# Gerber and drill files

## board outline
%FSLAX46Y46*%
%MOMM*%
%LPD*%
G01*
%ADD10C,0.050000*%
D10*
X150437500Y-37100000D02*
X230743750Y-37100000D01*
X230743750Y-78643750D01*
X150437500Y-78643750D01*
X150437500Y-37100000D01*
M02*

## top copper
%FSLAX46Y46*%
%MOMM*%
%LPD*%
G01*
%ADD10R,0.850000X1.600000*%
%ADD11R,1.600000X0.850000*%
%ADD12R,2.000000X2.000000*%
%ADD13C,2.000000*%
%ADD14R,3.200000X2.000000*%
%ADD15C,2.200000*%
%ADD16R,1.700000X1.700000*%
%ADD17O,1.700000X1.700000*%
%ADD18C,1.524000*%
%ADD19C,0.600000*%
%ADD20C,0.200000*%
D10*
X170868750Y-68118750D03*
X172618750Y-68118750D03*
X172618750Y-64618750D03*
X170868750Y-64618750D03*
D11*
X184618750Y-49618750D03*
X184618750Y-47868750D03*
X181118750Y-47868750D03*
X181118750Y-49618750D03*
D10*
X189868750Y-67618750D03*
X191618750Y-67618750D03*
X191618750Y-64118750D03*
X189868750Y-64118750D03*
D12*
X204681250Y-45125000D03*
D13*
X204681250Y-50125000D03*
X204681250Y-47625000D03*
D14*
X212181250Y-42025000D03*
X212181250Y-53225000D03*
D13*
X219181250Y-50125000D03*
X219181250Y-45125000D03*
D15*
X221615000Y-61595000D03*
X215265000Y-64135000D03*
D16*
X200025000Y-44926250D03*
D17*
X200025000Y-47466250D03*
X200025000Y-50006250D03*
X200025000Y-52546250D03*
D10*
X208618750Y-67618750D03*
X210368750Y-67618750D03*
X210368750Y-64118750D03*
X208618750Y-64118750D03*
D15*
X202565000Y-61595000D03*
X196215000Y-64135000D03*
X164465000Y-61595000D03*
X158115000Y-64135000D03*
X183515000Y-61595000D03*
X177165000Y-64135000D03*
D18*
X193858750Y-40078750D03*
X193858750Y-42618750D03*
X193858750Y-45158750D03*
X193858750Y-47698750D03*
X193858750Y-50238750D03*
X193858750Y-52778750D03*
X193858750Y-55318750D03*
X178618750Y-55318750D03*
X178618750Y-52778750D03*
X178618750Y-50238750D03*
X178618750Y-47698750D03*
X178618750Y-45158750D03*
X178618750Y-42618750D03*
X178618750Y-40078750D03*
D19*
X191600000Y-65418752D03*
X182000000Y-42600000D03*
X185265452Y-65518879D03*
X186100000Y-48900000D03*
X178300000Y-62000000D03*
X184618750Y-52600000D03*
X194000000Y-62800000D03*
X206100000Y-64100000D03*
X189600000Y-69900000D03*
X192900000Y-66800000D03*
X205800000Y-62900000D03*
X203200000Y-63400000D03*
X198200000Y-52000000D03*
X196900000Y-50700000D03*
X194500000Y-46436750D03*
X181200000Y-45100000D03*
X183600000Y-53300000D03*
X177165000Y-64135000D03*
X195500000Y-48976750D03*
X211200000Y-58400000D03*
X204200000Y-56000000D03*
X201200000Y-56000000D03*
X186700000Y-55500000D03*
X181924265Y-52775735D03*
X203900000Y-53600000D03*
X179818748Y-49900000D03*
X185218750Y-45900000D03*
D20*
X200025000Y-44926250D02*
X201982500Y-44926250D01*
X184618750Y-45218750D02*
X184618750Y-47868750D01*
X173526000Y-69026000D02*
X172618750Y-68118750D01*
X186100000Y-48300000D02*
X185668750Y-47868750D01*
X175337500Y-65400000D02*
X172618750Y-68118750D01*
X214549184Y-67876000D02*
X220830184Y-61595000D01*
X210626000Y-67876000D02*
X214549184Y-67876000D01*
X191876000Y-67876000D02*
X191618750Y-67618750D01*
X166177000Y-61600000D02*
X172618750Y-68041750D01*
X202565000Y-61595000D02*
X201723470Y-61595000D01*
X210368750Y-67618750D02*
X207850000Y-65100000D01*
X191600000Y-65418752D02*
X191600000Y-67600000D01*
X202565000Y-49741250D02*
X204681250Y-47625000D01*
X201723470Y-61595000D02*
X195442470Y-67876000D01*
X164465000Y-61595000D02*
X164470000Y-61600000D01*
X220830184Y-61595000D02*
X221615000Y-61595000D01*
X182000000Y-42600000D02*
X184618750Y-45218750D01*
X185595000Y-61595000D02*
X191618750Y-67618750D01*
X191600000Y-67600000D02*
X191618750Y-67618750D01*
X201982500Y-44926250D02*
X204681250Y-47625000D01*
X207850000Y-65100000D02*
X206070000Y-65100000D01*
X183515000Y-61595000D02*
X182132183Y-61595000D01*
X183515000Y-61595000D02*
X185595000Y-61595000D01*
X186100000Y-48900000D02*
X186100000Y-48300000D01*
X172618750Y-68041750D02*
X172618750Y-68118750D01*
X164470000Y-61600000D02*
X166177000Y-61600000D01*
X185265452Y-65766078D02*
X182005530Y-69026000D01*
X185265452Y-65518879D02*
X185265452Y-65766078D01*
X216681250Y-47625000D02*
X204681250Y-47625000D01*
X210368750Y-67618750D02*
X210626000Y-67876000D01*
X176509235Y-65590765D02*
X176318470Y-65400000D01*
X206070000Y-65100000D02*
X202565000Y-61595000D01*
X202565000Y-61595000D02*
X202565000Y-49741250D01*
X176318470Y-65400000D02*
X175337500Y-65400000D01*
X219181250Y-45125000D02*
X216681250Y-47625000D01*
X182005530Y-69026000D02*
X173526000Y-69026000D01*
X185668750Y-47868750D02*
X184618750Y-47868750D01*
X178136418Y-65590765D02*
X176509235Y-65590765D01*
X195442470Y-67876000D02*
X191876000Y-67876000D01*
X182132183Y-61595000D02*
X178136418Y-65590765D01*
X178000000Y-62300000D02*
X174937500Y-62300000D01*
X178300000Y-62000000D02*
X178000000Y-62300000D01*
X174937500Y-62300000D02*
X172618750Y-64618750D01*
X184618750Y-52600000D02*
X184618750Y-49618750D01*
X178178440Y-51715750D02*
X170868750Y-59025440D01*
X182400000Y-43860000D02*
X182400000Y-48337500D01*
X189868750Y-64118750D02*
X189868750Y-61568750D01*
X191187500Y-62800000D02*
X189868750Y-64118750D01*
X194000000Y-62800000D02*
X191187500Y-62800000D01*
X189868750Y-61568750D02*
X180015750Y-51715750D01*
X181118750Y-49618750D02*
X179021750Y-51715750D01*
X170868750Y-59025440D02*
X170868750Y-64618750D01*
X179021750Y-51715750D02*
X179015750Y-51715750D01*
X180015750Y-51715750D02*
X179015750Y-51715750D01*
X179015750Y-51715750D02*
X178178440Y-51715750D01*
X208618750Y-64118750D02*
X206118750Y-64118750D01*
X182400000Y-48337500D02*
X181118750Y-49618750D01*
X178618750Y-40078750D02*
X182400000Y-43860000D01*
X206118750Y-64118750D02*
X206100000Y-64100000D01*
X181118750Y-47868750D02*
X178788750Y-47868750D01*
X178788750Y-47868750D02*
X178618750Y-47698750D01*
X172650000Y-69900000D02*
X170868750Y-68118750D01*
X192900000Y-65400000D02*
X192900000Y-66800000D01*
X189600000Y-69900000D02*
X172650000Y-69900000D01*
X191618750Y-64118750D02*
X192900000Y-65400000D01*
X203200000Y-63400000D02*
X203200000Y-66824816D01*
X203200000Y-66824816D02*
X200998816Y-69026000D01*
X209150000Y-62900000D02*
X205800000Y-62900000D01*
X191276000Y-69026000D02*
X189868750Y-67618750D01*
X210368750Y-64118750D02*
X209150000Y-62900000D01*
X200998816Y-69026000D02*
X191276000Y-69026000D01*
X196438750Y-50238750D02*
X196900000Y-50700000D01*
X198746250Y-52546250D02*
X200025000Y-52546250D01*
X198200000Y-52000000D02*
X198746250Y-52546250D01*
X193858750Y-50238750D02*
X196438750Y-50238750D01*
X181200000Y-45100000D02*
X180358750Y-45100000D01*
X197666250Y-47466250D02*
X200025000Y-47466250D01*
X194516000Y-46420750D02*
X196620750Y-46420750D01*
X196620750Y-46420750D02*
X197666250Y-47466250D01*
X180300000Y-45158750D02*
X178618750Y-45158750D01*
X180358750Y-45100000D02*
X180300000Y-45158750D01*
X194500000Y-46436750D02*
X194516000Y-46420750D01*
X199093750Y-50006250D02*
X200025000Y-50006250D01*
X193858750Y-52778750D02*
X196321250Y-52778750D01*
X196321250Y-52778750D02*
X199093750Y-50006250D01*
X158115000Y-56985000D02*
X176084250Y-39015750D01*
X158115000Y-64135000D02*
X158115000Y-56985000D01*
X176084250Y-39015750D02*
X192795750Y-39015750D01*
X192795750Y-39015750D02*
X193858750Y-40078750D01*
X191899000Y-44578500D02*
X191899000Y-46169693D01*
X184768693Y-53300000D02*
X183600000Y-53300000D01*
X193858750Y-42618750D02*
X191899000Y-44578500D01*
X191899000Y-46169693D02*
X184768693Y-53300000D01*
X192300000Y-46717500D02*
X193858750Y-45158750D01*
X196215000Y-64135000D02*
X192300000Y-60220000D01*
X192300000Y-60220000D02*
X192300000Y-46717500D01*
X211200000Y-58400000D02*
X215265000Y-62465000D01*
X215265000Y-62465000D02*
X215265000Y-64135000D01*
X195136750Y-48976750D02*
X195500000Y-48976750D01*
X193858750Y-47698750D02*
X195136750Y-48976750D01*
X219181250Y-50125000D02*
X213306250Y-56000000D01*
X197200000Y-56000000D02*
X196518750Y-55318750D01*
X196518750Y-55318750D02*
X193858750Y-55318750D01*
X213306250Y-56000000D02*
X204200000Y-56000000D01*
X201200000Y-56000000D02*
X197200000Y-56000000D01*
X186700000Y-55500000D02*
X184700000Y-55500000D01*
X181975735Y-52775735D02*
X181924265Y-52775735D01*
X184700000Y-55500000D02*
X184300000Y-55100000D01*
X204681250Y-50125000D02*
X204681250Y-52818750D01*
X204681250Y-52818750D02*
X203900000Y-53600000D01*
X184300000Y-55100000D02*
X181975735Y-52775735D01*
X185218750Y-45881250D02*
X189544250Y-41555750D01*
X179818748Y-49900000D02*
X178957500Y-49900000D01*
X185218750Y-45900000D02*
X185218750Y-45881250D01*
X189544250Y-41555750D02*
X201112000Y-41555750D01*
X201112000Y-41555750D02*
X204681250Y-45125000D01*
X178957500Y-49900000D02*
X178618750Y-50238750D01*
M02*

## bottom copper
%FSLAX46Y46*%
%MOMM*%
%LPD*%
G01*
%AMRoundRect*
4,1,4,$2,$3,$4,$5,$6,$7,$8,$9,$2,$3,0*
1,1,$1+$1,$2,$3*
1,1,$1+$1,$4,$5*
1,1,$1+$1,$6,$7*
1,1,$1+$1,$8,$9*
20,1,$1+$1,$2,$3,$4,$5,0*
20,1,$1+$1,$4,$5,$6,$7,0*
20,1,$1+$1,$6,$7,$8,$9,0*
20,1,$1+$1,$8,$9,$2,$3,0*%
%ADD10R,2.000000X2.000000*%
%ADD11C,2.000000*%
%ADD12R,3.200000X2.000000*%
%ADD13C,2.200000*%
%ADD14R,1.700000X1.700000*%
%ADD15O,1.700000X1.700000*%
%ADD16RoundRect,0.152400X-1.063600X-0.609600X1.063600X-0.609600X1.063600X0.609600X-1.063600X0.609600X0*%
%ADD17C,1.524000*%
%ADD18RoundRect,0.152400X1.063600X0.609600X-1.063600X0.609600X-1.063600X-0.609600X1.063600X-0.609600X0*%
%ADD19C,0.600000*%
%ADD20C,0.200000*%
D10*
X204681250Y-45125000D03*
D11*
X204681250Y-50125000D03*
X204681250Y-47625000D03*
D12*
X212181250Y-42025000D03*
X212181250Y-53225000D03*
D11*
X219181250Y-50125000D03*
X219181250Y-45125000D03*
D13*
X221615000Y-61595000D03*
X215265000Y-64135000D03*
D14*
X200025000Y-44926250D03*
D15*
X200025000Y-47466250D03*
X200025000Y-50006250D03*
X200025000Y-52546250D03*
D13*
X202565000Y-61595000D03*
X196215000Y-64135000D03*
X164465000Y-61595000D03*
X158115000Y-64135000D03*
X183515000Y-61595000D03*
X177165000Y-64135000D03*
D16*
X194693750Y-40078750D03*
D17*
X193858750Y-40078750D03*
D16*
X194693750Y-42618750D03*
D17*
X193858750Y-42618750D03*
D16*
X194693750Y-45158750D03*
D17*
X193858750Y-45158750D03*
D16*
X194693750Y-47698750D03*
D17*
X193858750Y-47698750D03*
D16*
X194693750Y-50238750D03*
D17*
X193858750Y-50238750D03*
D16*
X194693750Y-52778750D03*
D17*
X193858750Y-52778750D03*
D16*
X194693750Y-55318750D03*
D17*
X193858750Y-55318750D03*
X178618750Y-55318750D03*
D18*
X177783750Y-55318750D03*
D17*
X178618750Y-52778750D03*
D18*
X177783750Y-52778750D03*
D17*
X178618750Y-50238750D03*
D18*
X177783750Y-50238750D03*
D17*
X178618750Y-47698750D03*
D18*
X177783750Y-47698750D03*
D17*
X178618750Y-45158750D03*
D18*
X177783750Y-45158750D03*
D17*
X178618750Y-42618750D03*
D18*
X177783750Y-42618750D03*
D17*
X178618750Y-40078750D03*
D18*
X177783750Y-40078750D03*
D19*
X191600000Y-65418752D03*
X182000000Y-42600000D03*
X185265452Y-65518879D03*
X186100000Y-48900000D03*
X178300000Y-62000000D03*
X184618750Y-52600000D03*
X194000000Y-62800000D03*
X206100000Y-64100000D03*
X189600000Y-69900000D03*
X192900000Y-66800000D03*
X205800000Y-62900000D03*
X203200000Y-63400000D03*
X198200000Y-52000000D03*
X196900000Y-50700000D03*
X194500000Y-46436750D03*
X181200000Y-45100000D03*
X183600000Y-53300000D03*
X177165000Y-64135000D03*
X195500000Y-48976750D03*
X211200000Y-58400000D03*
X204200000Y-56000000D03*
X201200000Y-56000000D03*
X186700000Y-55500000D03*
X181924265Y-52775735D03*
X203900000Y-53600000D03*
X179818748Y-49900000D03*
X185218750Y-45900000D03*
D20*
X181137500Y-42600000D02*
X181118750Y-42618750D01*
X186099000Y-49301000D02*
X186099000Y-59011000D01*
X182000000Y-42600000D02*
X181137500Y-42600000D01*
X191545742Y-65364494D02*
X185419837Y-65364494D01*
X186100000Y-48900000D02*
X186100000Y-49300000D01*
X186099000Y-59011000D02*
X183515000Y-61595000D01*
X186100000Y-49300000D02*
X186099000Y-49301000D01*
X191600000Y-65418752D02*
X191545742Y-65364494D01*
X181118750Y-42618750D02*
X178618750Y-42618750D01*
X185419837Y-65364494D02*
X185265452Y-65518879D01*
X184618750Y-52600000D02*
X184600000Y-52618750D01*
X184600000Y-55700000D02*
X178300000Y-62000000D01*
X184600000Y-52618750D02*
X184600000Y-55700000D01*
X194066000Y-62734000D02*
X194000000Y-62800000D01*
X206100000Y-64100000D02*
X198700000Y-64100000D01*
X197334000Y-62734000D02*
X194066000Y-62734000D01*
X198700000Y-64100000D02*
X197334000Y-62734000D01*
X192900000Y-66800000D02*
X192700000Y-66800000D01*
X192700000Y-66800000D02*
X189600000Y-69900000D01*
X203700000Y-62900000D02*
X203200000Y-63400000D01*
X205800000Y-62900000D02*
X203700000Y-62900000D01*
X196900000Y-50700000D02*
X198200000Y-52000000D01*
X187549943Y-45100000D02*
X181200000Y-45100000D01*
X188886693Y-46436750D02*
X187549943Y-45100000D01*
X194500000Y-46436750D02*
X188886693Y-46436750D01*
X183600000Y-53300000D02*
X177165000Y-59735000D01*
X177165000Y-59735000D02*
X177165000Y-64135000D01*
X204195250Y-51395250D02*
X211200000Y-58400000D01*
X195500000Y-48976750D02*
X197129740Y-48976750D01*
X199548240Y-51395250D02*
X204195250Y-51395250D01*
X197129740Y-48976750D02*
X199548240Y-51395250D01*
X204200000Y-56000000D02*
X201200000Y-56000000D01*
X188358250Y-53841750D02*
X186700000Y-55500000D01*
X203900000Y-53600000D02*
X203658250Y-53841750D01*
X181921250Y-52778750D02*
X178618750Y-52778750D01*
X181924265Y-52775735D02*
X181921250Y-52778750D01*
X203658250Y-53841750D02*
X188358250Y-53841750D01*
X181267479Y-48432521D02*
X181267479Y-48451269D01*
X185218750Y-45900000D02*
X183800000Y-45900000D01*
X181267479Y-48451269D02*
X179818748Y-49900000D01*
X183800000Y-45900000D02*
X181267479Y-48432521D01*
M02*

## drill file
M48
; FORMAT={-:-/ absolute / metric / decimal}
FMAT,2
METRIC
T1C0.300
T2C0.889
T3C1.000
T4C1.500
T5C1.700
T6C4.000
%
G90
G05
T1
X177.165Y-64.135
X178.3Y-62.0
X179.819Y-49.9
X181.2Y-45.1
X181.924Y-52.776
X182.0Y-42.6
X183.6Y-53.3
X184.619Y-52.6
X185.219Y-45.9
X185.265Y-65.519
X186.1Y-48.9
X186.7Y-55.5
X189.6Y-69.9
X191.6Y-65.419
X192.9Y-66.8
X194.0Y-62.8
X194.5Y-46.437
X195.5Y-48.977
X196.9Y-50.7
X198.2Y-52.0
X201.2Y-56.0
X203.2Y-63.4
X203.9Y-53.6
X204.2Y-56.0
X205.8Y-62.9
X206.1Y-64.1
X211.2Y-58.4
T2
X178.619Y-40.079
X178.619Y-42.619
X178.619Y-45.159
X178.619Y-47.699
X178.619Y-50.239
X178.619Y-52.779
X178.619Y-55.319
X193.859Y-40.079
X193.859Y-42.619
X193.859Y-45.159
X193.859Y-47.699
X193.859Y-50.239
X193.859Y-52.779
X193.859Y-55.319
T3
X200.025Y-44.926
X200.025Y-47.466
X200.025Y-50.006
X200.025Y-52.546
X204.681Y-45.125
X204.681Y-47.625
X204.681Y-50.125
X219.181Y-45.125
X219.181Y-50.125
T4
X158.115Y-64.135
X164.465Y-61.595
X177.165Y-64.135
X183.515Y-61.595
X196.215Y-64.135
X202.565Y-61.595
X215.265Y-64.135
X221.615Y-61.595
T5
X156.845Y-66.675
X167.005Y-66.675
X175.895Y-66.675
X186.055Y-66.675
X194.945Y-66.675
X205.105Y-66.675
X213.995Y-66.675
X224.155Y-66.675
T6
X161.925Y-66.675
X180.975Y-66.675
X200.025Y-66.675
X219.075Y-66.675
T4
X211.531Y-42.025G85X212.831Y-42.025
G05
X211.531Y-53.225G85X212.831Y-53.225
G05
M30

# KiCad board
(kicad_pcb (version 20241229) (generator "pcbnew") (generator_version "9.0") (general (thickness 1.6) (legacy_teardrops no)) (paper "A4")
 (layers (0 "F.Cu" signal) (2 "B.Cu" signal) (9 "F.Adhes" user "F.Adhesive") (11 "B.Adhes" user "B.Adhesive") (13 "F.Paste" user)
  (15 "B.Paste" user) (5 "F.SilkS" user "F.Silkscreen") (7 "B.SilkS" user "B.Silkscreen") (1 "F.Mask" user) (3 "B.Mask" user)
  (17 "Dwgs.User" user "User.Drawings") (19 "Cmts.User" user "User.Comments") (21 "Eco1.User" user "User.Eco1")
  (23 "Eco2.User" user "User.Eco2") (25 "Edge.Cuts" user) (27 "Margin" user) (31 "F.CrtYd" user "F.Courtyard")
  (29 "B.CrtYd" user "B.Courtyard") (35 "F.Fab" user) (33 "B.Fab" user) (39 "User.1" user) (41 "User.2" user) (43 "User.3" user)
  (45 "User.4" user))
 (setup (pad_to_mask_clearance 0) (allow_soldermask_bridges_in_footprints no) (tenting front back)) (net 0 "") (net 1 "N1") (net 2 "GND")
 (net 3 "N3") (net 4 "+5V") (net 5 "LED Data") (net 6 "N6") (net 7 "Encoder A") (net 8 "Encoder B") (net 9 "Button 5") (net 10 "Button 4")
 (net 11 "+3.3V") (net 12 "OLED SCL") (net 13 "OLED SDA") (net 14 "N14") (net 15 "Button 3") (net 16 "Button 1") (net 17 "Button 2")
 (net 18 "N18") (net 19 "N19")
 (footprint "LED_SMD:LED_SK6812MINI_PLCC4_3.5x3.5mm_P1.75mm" (layer "F.Cu") (at 171.74375 66.36875 90)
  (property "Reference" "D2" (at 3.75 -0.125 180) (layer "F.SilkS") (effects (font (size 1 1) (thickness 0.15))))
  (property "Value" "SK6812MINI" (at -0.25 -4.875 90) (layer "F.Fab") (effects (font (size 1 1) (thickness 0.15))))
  (pad "1" smd rect (at -1.75 -0.875 90) (size 1.6 0.85) (layers "F.Cu" "F.Mask" "F.Paste") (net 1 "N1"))
  (pad "2" smd rect (at -1.75 0.875 90) (size 1.6 0.85) (layers "F.Cu" "F.Mask" "F.Paste") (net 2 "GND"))
  (pad "3" smd rect (at 1.75 0.875 90) (size 1.6 0.85) (layers "F.Cu" "F.Mask" "F.Paste") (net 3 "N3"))
  (pad "4" smd rect (at 1.75 -0.875 90) (size 1.6 0.85) (layers "F.Cu" "F.Mask" "F.Paste") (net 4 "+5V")))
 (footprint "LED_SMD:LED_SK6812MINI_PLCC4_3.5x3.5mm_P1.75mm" (layer "F.Cu") (at 182.86875 48.74375 180)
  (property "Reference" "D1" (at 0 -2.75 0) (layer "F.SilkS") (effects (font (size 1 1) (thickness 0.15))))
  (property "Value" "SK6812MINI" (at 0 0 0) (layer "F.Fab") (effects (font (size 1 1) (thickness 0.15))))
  (pad "1" smd rect (at -1.75 -0.875 180) (size 1.6 0.85) (layers "F.Cu" "F.Mask" "F.Paste") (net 3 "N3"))
  (pad "2" smd rect (at -1.75 0.875 180) (size 1.6 0.85) (layers "F.Cu" "F.Mask" "F.Paste") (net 2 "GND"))
  (pad "3" smd rect (at 1.75 0.875 180) (size 1.6 0.85) (layers "F.Cu" "F.Mask" "F.Paste") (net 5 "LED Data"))
  (pad "4" smd rect (at 1.75 -0.875 180) (size 1.6 0.85) (layers "F.Cu" "F.Mask" "F.Paste") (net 4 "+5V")))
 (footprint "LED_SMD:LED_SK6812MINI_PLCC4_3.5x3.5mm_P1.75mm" (layer "F.Cu") (at 190.74375 65.86875 90)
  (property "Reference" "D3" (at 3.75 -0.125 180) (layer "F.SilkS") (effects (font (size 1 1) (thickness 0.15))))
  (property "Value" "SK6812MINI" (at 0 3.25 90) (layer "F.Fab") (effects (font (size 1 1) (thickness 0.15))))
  (pad "1" smd rect (at -1.75 -0.875 90) (size 1.6 0.85) (layers "F.Cu" "F.Mask" "F.Paste") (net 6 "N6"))
  (pad "2" smd rect (at -1.75 0.875 90) (size 1.6 0.85) (layers "F.Cu" "F.Mask" "F.Paste") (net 2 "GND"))
  (pad "3" smd rect (at 1.75 0.875 90) (size 1.6 0.85) (layers "F.Cu" "F.Mask" "F.Paste") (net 1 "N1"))
  (pad "4" smd rect (at 1.75 -0.875 90) (size 1.6 0.85) (layers "F.Cu" "F.Mask" "F.Paste") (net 4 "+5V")))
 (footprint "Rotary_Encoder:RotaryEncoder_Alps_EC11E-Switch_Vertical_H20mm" (layer "F.Cu") (at 204.68125 45.125)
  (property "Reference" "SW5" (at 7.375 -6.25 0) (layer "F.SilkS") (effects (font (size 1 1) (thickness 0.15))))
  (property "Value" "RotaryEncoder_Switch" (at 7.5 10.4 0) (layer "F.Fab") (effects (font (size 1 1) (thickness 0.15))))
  (pad "A" thru_hole rect (at 0 0) (size 2 2) (drill 1) (layers "*.Cu" "*.Mask") (remove_unused_layers no) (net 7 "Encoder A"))
  (pad "B" thru_hole circle (at 0 5) (size 2 2) (drill 1) (layers "*.Cu" "*.Mask") (remove_unused_layers no) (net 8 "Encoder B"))
  (pad "C" thru_hole circle (at 0 2.5) (size 2 2) (drill 1) (layers "*.Cu" "*.Mask") (remove_unused_layers no) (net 2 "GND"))
  (pad "MP" thru_hole rect (at 7.5 -3.1) (size 3.2 2) (drill oval 2.8 1.5) (layers "*.Cu" "*.Mask") (remove_unused_layers no))
  (pad "MP" thru_hole rect (at 7.5 8.1) (size 3.2 2) (drill oval 2.8 1.5) (layers "*.Cu" "*.Mask") (remove_unused_layers no))
  (pad "S1" thru_hole circle (at 14.5 5) (size 2 2) (drill 1) (layers "*.Cu" "*.Mask") (remove_unused_layers no) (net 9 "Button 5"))
  (pad "S2" thru_hole circle (at 14.5 0) (size 2 2) (drill 1) (layers "*.Cu" "*.Mask") (remove_unused_layers no) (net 2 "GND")))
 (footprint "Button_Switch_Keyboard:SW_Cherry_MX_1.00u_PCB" (layer "F.Cu") (at 221.615 61.595)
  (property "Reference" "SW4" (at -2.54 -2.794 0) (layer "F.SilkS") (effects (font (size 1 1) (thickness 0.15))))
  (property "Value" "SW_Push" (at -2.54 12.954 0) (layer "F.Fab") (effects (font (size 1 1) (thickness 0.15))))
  (pad "" np_thru_hole circle (at -7.62 5.08) (size 1.7 1.7) (drill 1.7) (layers "*.Cu" "*.Mask"))
  (pad "" np_thru_hole circle (at -2.54 5.08) (size 4 4) (drill 4) (layers "*.Cu" "*.Mask"))
  (pad "" np_thru_hole circle (at 2.54 5.08) (size 1.7 1.7) (drill 1.7) (layers "*.Cu" "*.Mask"))
  (pad "1" thru_hole circle (at 0 0) (size 2.2 2.2) (drill 1.5) (layers "*.Cu" "*.Mask") (remove_unused_layers no) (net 2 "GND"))
  (pad "2" thru_hole circle (at -6.35 2.54) (size 2.2 2.2) (drill 1.5) (layers "*.Cu" "*.Mask") (remove_unused_layers no)
   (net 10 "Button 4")))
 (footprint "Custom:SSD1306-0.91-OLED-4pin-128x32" (layer "F.Cu") (at 163.525 42.73625)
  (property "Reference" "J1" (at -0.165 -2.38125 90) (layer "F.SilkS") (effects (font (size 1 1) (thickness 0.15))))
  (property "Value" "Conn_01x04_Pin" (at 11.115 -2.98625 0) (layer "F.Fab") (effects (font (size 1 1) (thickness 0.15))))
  (pad "1" thru_hole rect (at 36.5 2.19) (size 1.7 1.7) (drill 1) (layers "*.Cu" "*.Mask") (remove_unused_layers no) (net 2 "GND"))
  (pad "2" thru_hole oval (at 36.5 4.73) (size 1.7 1.7) (drill 1) (layers "*.Cu" "*.Mask") (remove_unused_layers no) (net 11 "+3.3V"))
  (pad "3" thru_hole oval (at 36.5 7.27) (size 1.7 1.7) (drill 1) (layers "*.Cu" "*.Mask") (remove_unused_layers no) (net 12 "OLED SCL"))
  (pad "4" thru_hole oval (at 36.5 9.81) (size 1.7 1.7) (drill 1) (layers "*.Cu" "*.Mask") (remove_unused_layers no) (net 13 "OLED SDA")))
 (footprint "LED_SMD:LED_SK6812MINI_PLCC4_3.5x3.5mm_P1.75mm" (layer "F.Cu") (at 209.49375 65.86875 90)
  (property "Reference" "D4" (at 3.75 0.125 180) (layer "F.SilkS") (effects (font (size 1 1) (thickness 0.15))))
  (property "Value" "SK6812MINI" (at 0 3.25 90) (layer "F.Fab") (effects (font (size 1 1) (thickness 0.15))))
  (pad "1" smd rect (at -1.75 -0.875 90) (size 1.6 0.85) (layers "F.Cu" "F.Mask" "F.Paste") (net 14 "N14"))
  (pad "2" smd rect (at -1.75 0.875 90) (size 1.6 0.85) (layers "F.Cu" "F.Mask" "F.Paste") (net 2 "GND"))
  (pad "3" smd rect (at 1.75 0.875 90) (size 1.6 0.85) (layers "F.Cu" "F.Mask" "F.Paste") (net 6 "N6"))
  (pad "4" smd rect (at 1.75 -0.875 90) (size 1.6 0.85) (layers "F.Cu" "F.Mask" "F.Paste") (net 4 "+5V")))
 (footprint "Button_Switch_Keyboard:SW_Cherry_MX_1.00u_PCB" (layer "F.Cu") (at 202.565 61.595)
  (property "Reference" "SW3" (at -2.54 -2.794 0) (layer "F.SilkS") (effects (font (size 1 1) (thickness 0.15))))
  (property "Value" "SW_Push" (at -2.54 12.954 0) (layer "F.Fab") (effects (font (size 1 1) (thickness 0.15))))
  (pad "" np_thru_hole circle (at -7.62 5.08) (size 1.7 1.7) (drill 1.7) (layers "*.Cu" "*.Mask"))
  (pad "" np_thru_hole circle (at -2.54 5.08) (size 4 4) (drill 4) (layers "*.Cu" "*.Mask"))
  (pad "" np_thru_hole circle (at 2.54 5.08) (size 1.7 1.7) (drill 1.7) (layers "*.Cu" "*.Mask"))
  (pad "1" thru_hole circle (at 0 0) (size 2.2 2.2) (drill 1.5) (layers "*.Cu" "*.Mask") (remove_unused_layers no) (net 2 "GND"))
  (pad "2" thru_hole circle (at -6.35 2.54) (size 2.2 2.2) (drill 1.5) (layers "*.Cu" "*.Mask") (remove_unused_layers no)
   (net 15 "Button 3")))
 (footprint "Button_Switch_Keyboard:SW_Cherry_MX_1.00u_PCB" (layer "F.Cu") (at 164.465 61.595)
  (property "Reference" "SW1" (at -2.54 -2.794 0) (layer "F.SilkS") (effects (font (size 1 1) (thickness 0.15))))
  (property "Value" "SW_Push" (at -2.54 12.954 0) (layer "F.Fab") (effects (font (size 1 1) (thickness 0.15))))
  (pad "" np_thru_hole circle (at -7.62 5.08) (size 1.7 1.7) (drill 1.7) (layers "*.Cu" "*.Mask"))
  (pad "" np_thru_hole circle (at -2.54 5.08) (size 4 4) (drill 4) (layers "*.Cu" "*.Mask"))
  (pad "" np_thru_hole circle (at 2.54 5.08) (size 1.7 1.7) (drill 1.7) (layers "*.Cu" "*.Mask"))
  (pad "1" thru_hole circle (at 0 0) (size 2.2 2.2) (drill 1.5) (layers "*.Cu" "*.Mask") (remove_unused_layers no) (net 2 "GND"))
  (pad "2" thru_hole circle (at -6.35 2.54) (size 2.2 2.2) (drill 1.5) (layers "*.Cu" "*.Mask") (remove_unused_layers no)
   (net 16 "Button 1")))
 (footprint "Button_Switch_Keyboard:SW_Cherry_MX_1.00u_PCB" (layer "F.Cu") (at 183.515 61.595)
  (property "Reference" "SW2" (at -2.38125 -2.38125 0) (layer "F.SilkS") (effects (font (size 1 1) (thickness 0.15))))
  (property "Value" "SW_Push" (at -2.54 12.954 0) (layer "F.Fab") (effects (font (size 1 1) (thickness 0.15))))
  (pad "" np_thru_hole circle (at -7.62 5.08) (size 1.7 1.7) (drill 1.7) (layers "*.Cu" "*.Mask"))
  (pad "" np_thru_hole circle (at -2.54 5.08) (size 4 4) (drill 4) (layers "*.Cu" "*.Mask"))
  (pad "" np_thru_hole circle (at 2.54 5.08) (size 1.7 1.7) (drill 1.7) (layers "*.Cu" "*.Mask"))
  (pad "1" thru_hole circle (at 0 0) (size 2.2 2.2) (drill 1.5) (layers "*.Cu" "*.Mask") (remove_unused_layers no) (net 2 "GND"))
  (pad "2" thru_hole circle (at -6.35 2.54) (size 2.2 2.2) (drill 1.5) (layers "*.Cu" "*.Mask") (remove_unused_layers no)
   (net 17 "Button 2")))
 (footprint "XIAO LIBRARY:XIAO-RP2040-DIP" (layer "B.Cu") (at 186.23875 47.69875 180)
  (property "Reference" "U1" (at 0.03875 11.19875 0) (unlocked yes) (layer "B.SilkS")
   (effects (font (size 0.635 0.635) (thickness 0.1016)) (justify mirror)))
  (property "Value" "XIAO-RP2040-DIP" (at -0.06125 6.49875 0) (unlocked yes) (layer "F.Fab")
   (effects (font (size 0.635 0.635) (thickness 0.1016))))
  (pad "1" smd roundrect (at -8.455 7.62) (size 2.432 1.524) (layers "B.Cu" "B.Mask") (roundrect_rratio 0.1) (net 16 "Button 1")
   (thermal_bridge_angle 45))
  (pad "1" thru_hole circle (at -7.62 7.62) (size 1.524 1.524) (drill 0.889) (layers "*.Cu" "*.Mask") (remove_unused_layers no)
   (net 16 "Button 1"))
  (pad "2" smd roundrect (at -8.455 5.08) (size 2.432 1.524) (layers "B.Cu" "B.Mask") (roundrect_rratio 0.1) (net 17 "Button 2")
   (thermal_bridge_angle 45))
  (pad "2" thru_hole circle (at -7.62 5.08) (size 1.524 1.524) (drill 0.889) (layers "*.Cu" "*.Mask") (remove_unused_layers no)
   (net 17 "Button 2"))
  (pad "3" smd roundrect (at -8.455 2.54) (size 2.432 1.524) (layers "B.Cu" "B.Mask") (roundrect_rratio 0.1) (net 15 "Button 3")
   (thermal_bridge_angle 45))
  (pad "3" thru_hole circle (at -7.62 2.54) (size 1.524 1.524) (drill 0.889) (layers "*.Cu" "*.Mask") (remove_unused_layers no)
   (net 15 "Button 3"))
  (pad "4" smd roundrect (at -8.455 0) (size 2.432 1.524) (layers "B.Cu" "B.Mask") (roundrect_rratio 0.1) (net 10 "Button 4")
   (thermal_bridge_angle 45))
  (pad "4" thru_hole circle (at -7.62 0) (size 1.524 1.524) (drill 0.889) (layers "*.Cu" "*.Mask") (remove_unused_layers no)
   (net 10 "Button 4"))
  (pad "5" smd roundrect (at -8.455 -2.54) (size 2.432 1.524) (layers "B.Cu" "B.Mask") (roundrect_rratio 0.1) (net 13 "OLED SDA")
   (thermal_bridge_angle 45))
  (pad "5" thru_hole circle (at -7.62 -2.54) (size 1.524 1.524) (drill 0.889) (layers "*.Cu" "*.Mask") (remove_unused_layers no)
   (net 13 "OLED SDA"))
  (pad "6" smd roundrect (at -8.455 -5.08) (size 2.432 1.524) (layers "B.Cu" "B.Mask") (roundrect_rratio 0.1) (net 12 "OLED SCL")
   (thermal_bridge_angle 45))
  (pad "6" thru_hole circle (at -7.62 -5.08) (size 1.524 1.524) (drill 0.889) (layers "*.Cu" "*.Mask") (remove_unused_layers no)
   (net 12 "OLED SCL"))
  (pad "7" smd roundrect (at -8.455 -7.62) (size 2.432 1.524) (layers "B.Cu" "B.Mask") (roundrect_rratio 0.1) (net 9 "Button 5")
   (thermal_bridge_angle 45))
  (pad "7" thru_hole circle (at -7.62 -7.62) (size 1.524 1.524) (drill 0.889) (layers "*.Cu" "*.Mask") (remove_unused_layers no)
   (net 9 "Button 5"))
  (pad "8" thru_hole circle (at 7.62 -7.62 180) (size 1.524 1.524) (drill 0.889) (layers "*.Cu" "*.Mask") (remove_unused_layers no)
   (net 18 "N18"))
  (pad "8" smd roundrect (at 8.455 -7.62 180) (size 2.432 1.524) (layers "B.Cu" "B.Mask") (roundrect_rratio 0.1) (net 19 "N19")
   (thermal_bridge_angle 45))
  (pad "9" thru_hole circle (at 7.62 -5.08 180) (size 1.524 1.524) (drill 0.889) (layers "*.Cu" "*.Mask") (remove_unused_layers no)
   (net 8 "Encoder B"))
  (pad "9" smd roundrect (at 8.455 -5.08 180) (size 2.432 1.524) (layers "B.Cu" "B.Mask") (roundrect_rratio 0.1) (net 8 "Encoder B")
   (thermal_bridge_angle 45))
  (pad "10" thru_hole circle (at 7.62 -2.54 180) (size 1.524 1.524) (drill 0.889) (layers "*.Cu" "*.Mask") (remove_unused_layers no)
   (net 7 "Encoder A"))
  (pad "10" smd roundrect (at 8.455 -2.54 180) (size 2.432 1.524) (layers "B.Cu" "B.Mask") (roundrect_rratio 0.1) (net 7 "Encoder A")
   (thermal_bridge_angle 45))
  (pad "11" thru_hole circle (at 7.62 0 180) (size 1.524 1.524) (drill 0.889) (layers "*.Cu" "*.Mask") (remove_unused_layers no)
   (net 5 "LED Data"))
  (pad "11" smd roundrect (at 8.455 0 180) (size 2.432 1.524) (layers "B.Cu" "B.Mask") (roundrect_rratio 0.1) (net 5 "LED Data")
   (thermal_bridge_angle 45))
  (pad "12" thru_hole circle (at 7.62 2.54 180) (size 1.524 1.524) (drill 0.889) (layers "*.Cu" "*.Mask") (remove_unused_layers no)
   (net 11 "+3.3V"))
  (pad "12" smd roundrect (at 8.455 2.54 180) (size 2.432 1.524) (layers "B.Cu" "B.Mask") (roundrect_rratio 0.1) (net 11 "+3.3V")
   (thermal_bridge_angle 45))
  (pad "13" thru_hole circle (at 7.62 5.08 180) (size 1.524 1.524) (drill 0.889) (layers "*.Cu" "*.Mask") (remove_unused_layers no)
   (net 2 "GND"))
  (pad "13" smd roundrect (at 8.455 5.08 180) (size 2.432 1.524) (layers "B.Cu" "B.Mask") (roundrect_rratio 0.1) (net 2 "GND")
   (thermal_bridge_angle 45))
  (pad "14" thru_hole circle (at 7.62 7.62 180) (size 1.524 1.524) (drill 0.889) (layers "*.Cu" "*.Mask") (remove_unused_layers no)
   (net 4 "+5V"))
  (pad "14" smd roundrect (at 8.455 7.62 180) (size 2.432 1.524) (layers "B.Cu" "B.Mask") (roundrect_rratio 0.1) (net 4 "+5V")
   (thermal_bridge_angle 45)))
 (gr_rect (start 150.4375 37.1) (end 230.74375 78.64375) (stroke (width 0.05) (type default)) (fill no) (layer "Edge.Cuts"))
 (segment (start 200.025 44.92625) (end 201.9825 44.92625) (width 0.2) (layer "F.Cu") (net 2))
 (segment (start 184.61875 45.21875) (end 184.61875 47.86875) (width 0.2) (layer "F.Cu") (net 2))
 (segment (start 173.526 69.026) (end 172.61875 68.11875) (width 0.2) (layer "F.Cu") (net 2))
 (segment (start 186.1 48.3) (end 185.66875 47.86875) (width 0.2) (layer "F.Cu") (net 2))
 (segment (start 175.3375 65.4) (end 172.61875 68.11875) (width 0.2) (layer "F.Cu") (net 2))
 (segment (start 214.549184 67.876) (end 220.830184 61.595) (width 0.2) (layer "F.Cu") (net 2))
 (segment (start 210.626 67.876) (end 214.549184 67.876) (width 0.2) (layer "F.Cu") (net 2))
 (segment (start 191.876 67.876) (end 191.61875 67.61875) (width 0.2) (layer "F.Cu") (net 2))
 (segment (start 166.177 61.6) (end 172.61875 68.04175) (width 0.2) (layer "F.Cu") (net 2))
 (segment (start 202.565 61.595) (end 201.72347 61.595) (width 0.2) (layer "F.Cu") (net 2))
 (segment (start 210.36875 67.61875) (end 207.85 65.1) (width 0.2) (layer "F.Cu") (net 2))
 (segment (start 191.6 65.418752) (end 191.6 67.6) (width 0.2) (layer "F.Cu") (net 2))
 (segment (start 202.565 49.74125) (end 204.68125 47.625) (width 0.2) (layer "F.Cu") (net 2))
 (segment (start 201.72347 61.595) (end 195.44247 67.876) (width 0.2) (layer "F.Cu") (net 2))
 (segment (start 164.465 61.595) (end 164.47 61.6) (width 0.2) (layer "F.Cu") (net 2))
 (segment (start 220.830184 61.595) (end 221.615 61.595) (width 0.2) (layer "F.Cu") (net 2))
 (segment (start 182 42.6) (end 184.61875 45.21875) (width 0.2) (layer "F.Cu") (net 2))
 (segment (start 185.595 61.595) (end 191.61875 67.61875) (width 0.2) (layer "F.Cu") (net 2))
 (segment (start 191.6 67.6) (end 191.61875 67.61875) (width 0.2) (layer "F.Cu") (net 2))
 (segment (start 201.9825 44.92625) (end 204.68125 47.625) (width 0.2) (layer "F.Cu") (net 2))
 (segment (start 207.85 65.1) (end 206.07 65.1) (width 0.2) (layer "F.Cu") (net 2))
 (segment (start 183.515 61.595) (end 182.132183 61.595) (width 0.2) (layer "F.Cu") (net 2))
 (segment (start 183.515 61.595) (end 185.595 61.595) (width 0.2) (layer "F.Cu") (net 2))
 (segment (start 186.1 48.9) (end 186.1 48.3) (width 0.2) (layer "F.Cu") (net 2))
 (segment (start 172.61875 68.04175) (end 172.61875 68.11875) (width 0.2) (layer "F.Cu") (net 2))
 (segment (start 164.47 61.6) (end 166.177 61.6) (width 0.2) (layer "F.Cu") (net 2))
 (segment (start 185.265452 65.766078) (end 182.00553 69.026) (width 0.2) (layer "F.Cu") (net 2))
 (segment (start 185.265452 65.518879) (end 185.265452 65.766078) (width 0.2) (layer "F.Cu") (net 2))
 (segment (start 216.68125 47.625) (end 204.68125 47.625) (width 0.2) (layer "F.Cu") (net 2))
 (segment (start 210.36875 67.61875) (end 210.626 67.876) (width 0.2) (layer "F.Cu") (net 2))
 (segment (start 176.509235 65.590765) (end 176.31847 65.4) (width 0.2) (layer "F.Cu") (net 2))
 (segment (start 206.07 65.1) (end 202.565 61.595) (width 0.2) (layer "F.Cu") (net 2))
 (segment (start 202.565 61.595) (end 202.565 49.74125) (width 0.2) (layer "F.Cu") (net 2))
 (segment (start 176.31847 65.4) (end 175.3375 65.4) (width 0.2) (layer "F.Cu") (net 2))
 (segment (start 219.18125 45.125) (end 216.68125 47.625) (width 0.2) (layer "F.Cu") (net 2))
 (segment (start 182.00553 69.026) (end 173.526 69.026) (width 0.2) (layer "F.Cu") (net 2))
 (segment (start 185.66875 47.86875) (end 184.61875 47.86875) (width 0.2) (layer "F.Cu") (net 2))
 (segment (start 178.136418 65.590765) (end 176.509235 65.590765) (width 0.2) (layer "F.Cu") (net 2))
 (segment (start 195.44247 67.876) (end 191.876 67.876) (width 0.2) (layer "F.Cu") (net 2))
 (segment (start 182.132183 61.595) (end 178.136418 65.590765) (width 0.2) (layer "F.Cu") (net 2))
 (via (at 191.6 65.418752) (size 0.6) (drill 0.3) (layers "F.Cu" "B.Cu") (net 2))
 (via (at 182 42.6) (size 0.6) (drill 0.3) (layers "F.Cu" "B.Cu") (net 2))
 (via (at 185.265452 65.518879) (size 0.6) (drill 0.3) (layers "F.Cu" "B.Cu") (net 2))
 (via (at 186.1 48.9) (size 0.6) (drill 0.3) (layers "F.Cu" "B.Cu") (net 2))
 (segment (start 181.1375 42.6) (end 181.11875 42.61875) (width 0.2) (layer "B.Cu") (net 2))
 (segment (start 186.099 49.301) (end 186.099 59.011) (width 0.2) (layer "B.Cu") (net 2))
 (segment (start 182 42.6) (end 181.1375 42.6) (width 0.2) (layer "B.Cu") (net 2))
 (segment (start 191.545742 65.364494) (end 185.419837 65.364494) (width 0.2) (layer "B.Cu") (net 2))
 (segment (start 186.1 48.9) (end 186.1 49.3) (width 0.2) (layer "B.Cu") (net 2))
 (segment (start 186.099 59.011) (end 183.515 61.595) (width 0.2) (layer "B.Cu") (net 2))
 (segment (start 186.1 49.3) (end 186.099 49.301) (width 0.2) (layer "B.Cu") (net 2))
 (segment (start 191.6 65.418752) (end 191.545742 65.364494) (width 0.2) (layer "B.Cu") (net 2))
 (segment (start 181.11875 42.61875) (end 178.61875 42.61875) (width 0.2) (layer "B.Cu") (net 2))
 (segment (start 185.419837 65.364494) (end 185.265452 65.518879) (width 0.2) (layer "B.Cu") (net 2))
 (segment (start 178 62.3) (end 174.9375 62.3) (width 0.2) (layer "F.Cu") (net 3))
 (segment (start 178.3 62) (end 178 62.3) (width 0.2) (layer "F.Cu") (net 3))
 (segment (start 174.9375 62.3) (end 172.61875 64.61875) (width 0.2) (layer "F.Cu") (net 3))
 (segment (start 184.61875 52.6) (end 184.61875 49.61875) (width 0.2) (layer "F.Cu") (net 3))
 (via (at 178.3 62) (size 0.6) (drill 0.3) (layers "F.Cu" "B.Cu") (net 3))
 (via (at 184.61875 52.6) (size 0.6) (drill 0.3) (layers "F.Cu" "B.Cu") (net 3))
 (segment (start 184.61875 52.6) (end 184.6 52.61875) (width 0.2) (layer "B.Cu") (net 3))
 (segment (start 184.6 55.7) (end 178.3 62) (width 0.2) (layer "B.Cu") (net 3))
 (segment (start 184.6 52.61875) (end 184.6 55.7) (width 0.2) (layer "B.Cu") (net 3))
 (segment (start 178.17844 51.71575) (end 170.86875 59.02544) (width 0.2) (layer "F.Cu") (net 4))
 (segment (start 182.4 43.86) (end 182.4 48.3375) (width 0.2) (layer "F.Cu") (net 4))
 (segment (start 189.86875 64.11875) (end 189.86875 61.56875) (width 0.2) (layer "F.Cu") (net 4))
 (segment (start 191.1875 62.8) (end 189.86875 64.11875) (width 0.2) (layer "F.Cu") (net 4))
 (segment (start 194 62.8) (end 191.1875 62.8) (width 0.2) (layer "F.Cu") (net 4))
 (segment (start 189.86875 61.56875) (end 180.01575 51.71575) (width 0.2) (layer "F.Cu") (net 4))
 (segment (start 181.11875 49.61875) (end 179.02175 51.71575) (width 0.2) (layer "F.Cu") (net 4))
 (segment (start 170.86875 59.02544) (end 170.86875 64.61875) (width 0.2) (layer "F.Cu") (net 4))
 (segment (start 179.02175 51.71575) (end 179.01575 51.71575) (width 0.2) (layer "F.Cu") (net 4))
 (segment (start 180.01575 51.71575) (end 179.01575 51.71575) (width 0.2) (layer "F.Cu") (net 4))
 (segment (start 179.01575 51.71575) (end 178.17844 51.71575) (width 0.2) (layer "F.Cu") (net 4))
 (segment (start 208.61875 64.11875) (end 206.11875 64.11875) (width 0.2) (layer "F.Cu") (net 4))
 (segment (start 182.4 48.3375) (end 181.11875 49.61875) (width 0.2) (layer "F.Cu") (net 4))
 (segment (start 178.61875 40.07875) (end 182.4 43.86) (width 0.2) (layer "F.Cu") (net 4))
 (segment (start 206.11875 64.11875) (end 206.1 64.1) (width 0.2) (layer "F.Cu") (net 4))
 (via (at 194 62.8) (size 0.6) (drill 0.3) (layers "F.Cu" "B.Cu") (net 4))
 (via (at 206.1 64.1) (size 0.6) (drill 0.3) (layers "F.Cu" "B.Cu") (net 4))
 (segment (start 194.066 62.734) (end 194 62.8) (width 0.2) (layer "B.Cu") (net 4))
 (segment (start 206.1 64.1) (end 198.7 64.1) (width 0.2) (layer "B.Cu") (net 4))
 (segment (start 197.334 62.734) (end 194.066 62.734) (width 0.2) (layer "B.Cu") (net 4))
 (segment (start 198.7 64.1) (end 197.334 62.734) (width 0.2) (layer "B.Cu") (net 4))
 (segment (start 181.11875 47.86875) (end 178.78875 47.86875) (width 0.2) (layer "F.Cu") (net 5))
 (segment (start 178.78875 47.86875) (end 178.61875 47.69875) (width 0.2) (layer "F.Cu") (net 5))
 (segment (start 172.65 69.9) (end 170.86875 68.11875) (width 0.2) (layer "F.Cu") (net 1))
 (segment (start 192.9 65.4) (end 192.9 66.8) (width 0.2) (layer "F.Cu") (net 1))
 (segment (start 189.6 69.9) (end 172.65 69.9) (width 0.2) (layer "F.Cu") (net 1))
 (segment (start 191.61875 64.11875) (end 192.9 65.4) (width 0.2) (layer "F.Cu") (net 1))
 (via (at 189.6 69.9) (size 0.6) (drill 0.3) (layers "F.Cu" "B.Cu") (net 1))
 (via (at 192.9 66.8) (size 0.6) (drill 0.3) (layers "F.Cu" "B.Cu") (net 1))
 (segment (start 192.9 66.8) (end 192.7 66.8) (width 0.2) (layer "B.Cu") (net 1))
 (segment (start 192.7 66.8) (end 189.6 69.9) (width 0.2) (layer "B.Cu") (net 1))
 (segment (start 203.2 63.4) (end 203.2 66.824816) (width 0.2) (layer "F.Cu") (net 6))
 (segment (start 203.2 66.824816) (end 200.998816 69.026) (width 0.2) (layer "F.Cu") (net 6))
 (segment (start 209.15 62.9) (end 205.8 62.9) (width 0.2) (layer "F.Cu") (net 6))
 (segment (start 191.276 69.026) (end 189.86875 67.61875) (width 0.2) (layer "F.Cu") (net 6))
 (segment (start 210.36875 64.11875) (end 209.15 62.9) (width 0.2) (layer "F.Cu") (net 6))
 (segment (start 200.998816 69.026) (end 191.276 69.026) (width 0.2) (layer "F.Cu") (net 6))
 (via (at 205.8 62.9) (size 0.6) (drill 0.3) (layers "F.Cu" "B.Cu") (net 6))
 (via (at 203.2 63.4) (size 0.6) (drill 0.3) (layers "F.Cu" "B.Cu") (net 6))
 (segment (start 203.7 62.9) (end 203.2 63.4) (width 0.2) (layer "B.Cu") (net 6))
 (segment (start 205.8 62.9) (end 203.7 62.9) (width 0.2) (layer "B.Cu") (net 6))
 (segment (start 196.43875 50.23875) (end 196.9 50.7) (width 0.2) (layer "F.Cu") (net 13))
 (segment (start 198.74625 52.54625) (end 200.025 52.54625) (width 0.2) (layer "F.Cu") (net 13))
 (segment (start 198.2 52) (end 198.74625 52.54625) (width 0.2) (layer "F.Cu") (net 13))
 (segment (start 193.85875 50.23875) (end 196.43875 50.23875) (width 0.2) (layer "F.Cu") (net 13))
 (via (at 198.2 52) (size 0.6) (drill 0.3) (layers "F.Cu" "B.Cu") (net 13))
 (via (at 196.9 50.7) (size 0.6) (drill 0.3) (layers "F.Cu" "B.Cu") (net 13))
 (segment (start 196.9 50.7) (end 198.2 52) (width 0.2) (layer "B.Cu") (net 13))
 (segment (start 181.2 45.1) (end 180.35875 45.1) (width 0.2) (layer "F.Cu") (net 11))
 (segment (start 197.66625 47.46625) (end 200.025 47.46625) (width 0.2) (layer "F.Cu") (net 11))
 (segment (start 194.516 46.42075) (end 196.62075 46.42075) (width 0.2) (layer "F.Cu") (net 11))
 (segment (start 196.62075 46.42075) (end 197.66625 47.46625) (width 0.2) (layer "F.Cu") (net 11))
 (segment (start 180.3 45.15875) (end 178.61875 45.15875) (width 0.2) (layer "F.Cu") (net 11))
 (segment (start 180.35875 45.1) (end 180.3 45.15875) (width 0.2) (layer "F.Cu") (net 11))
 (segment (start 194.5 46.43675) (end 194.516 46.42075) (width 0.2) (layer "F.Cu") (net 11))
 (via (at 194.5 46.43675) (size 0.6) (drill 0.3) (layers "F.Cu" "B.Cu") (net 11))
 (via (at 181.2 45.1) (size 0.6) (drill 0.3) (layers "F.Cu" "B.Cu") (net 11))
 (segment (start 187.549943 45.1) (end 181.2 45.1) (width 0.2) (layer "B.Cu") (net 11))
 (segment (start 188.886693 46.43675) (end 187.549943 45.1) (width 0.2) (layer "B.Cu") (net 11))
 (segment (start 194.5 46.43675) (end 188.886693 46.43675) (width 0.2) (layer "B.Cu") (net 11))
 (segment (start 199.09375 50.00625) (end 200.025 50.00625) (width 0.2) (layer "F.Cu") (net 12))
 (segment (start 193.85875 52.77875) (end 196.32125 52.77875) (width 0.2) (layer "F.Cu") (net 12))
 (segment (start 196.32125 52.77875) (end 199.09375 50.00625) (width 0.2) (layer "F.Cu") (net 12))
 (segment (start 158.115 56.985) (end 176.08425 39.01575) (width 0.2) (layer "F.Cu") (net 16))
 (segment (start 158.115 64.135) (end 158.115 56.985) (width 0.2) (layer "F.Cu") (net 16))
 (segment (start 176.08425 39.01575) (end 192.79575 39.01575) (width 0.2) (layer "F.Cu") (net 16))
 (segment (start 192.79575 39.01575) (end 193.85875 40.07875) (width 0.2) (layer "F.Cu") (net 16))
 (segment (start 191.899 44.5785) (end 191.899 46.169693) (width 0.2) (layer "F.Cu") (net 17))
 (segment (start 184.768693 53.3) (end 183.6 53.3) (width 0.2) (layer "F.Cu") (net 17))
 (segment (start 193.85875 42.61875) (end 191.899 44.5785) (width 0.2) (layer "F.Cu") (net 17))
 (segment (start 191.899 46.169693) (end 184.768693 53.3) (width 0.2) (layer "F.Cu") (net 17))
 (via (at 183.6 53.3) (size 0.6) (drill 0.3) (layers "F.Cu" "B.Cu") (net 17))
 (via (at 177.165 64.135) (size 0.6) (drill 0.3) (layers "F.Cu" "B.Cu") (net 17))
 (segment (start 183.6 53.3) (end 177.165 59.735) (width 0.2) (layer "B.Cu") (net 17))
 (segment (start 177.165 59.735) (end 177.165 64.135) (width 0.2) (layer "B.Cu") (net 17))
 (segment (start 192.3 46.7175) (end 193.85875 45.15875) (width 0.2) (layer "F.Cu") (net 15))
 (segment (start 196.215 64.135) (end 192.3 60.22) (width 0.2) (layer "F.Cu") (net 15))
 (segment (start 192.3 60.22) (end 192.3 46.7175) (width 0.2) (layer "F.Cu") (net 15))
 (segment (start 211.2 58.4) (end 215.265 62.465) (width 0.2) (layer "F.Cu") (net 10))
 (segment (start 215.265 62.465) (end 215.265 64.135) (width 0.2) (layer "F.Cu") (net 10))
 (segment (start 195.13675 48.97675) (end 195.5 48.97675) (width 0.2) (layer "F.Cu") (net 10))
 (segment (start 193.85875 47.69875) (end 195.13675 48.97675) (width 0.2) (layer "F.Cu") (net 10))
 (via (at 195.5 48.97675) (size 0.6) (drill 0.3) (layers "F.Cu" "B.Cu") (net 10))
 (via (at 211.2 58.4) (size 0.6) (drill 0.3) (layers "F.Cu" "B.Cu") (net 10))
 (segment (start 204.19525 51.39525) (end 211.2 58.4) (width 0.2) (layer "B.Cu") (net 10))
 (segment (start 195.5 48.97675) (end 197.12974 48.97675) (width 0.2) (layer "B.Cu") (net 10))
 (segment (start 199.54824 51.39525) (end 204.19525 51.39525) (width 0.2) (layer "B.Cu") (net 10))
 (segment (start 197.12974 48.97675) (end 199.54824 51.39525) (width 0.2) (layer "B.Cu") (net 10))
 (segment (start 219.18125 50.125) (end 213.30625 56) (width 0.2) (layer "F.Cu") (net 9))
 (segment (start 197.2 56) (end 196.51875 55.31875) (width 0.2) (layer "F.Cu") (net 9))
 (segment (start 196.51875 55.31875) (end 193.85875 55.31875) (width 0.2) (layer "F.Cu") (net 9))
 (segment (start 213.30625 56) (end 204.2 56) (width 0.2) (layer "F.Cu") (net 9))
 (segment (start 201.2 56) (end 197.2 56) (width 0.2) (layer "F.Cu") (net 9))
 (via (at 204.2 56) (size 0.6) (drill 0.3) (layers "F.Cu" "B.Cu") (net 9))
 (via (at 201.2 56) (size 0.6) (drill 0.3) (layers "F.Cu" "B.Cu") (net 9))
 (segment (start 204.2 56) (end 201.2 56) (width 0.2) (layer "B.Cu") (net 9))
 (segment (start 186.7 55.5) (end 184.7 55.5) (width 0.2) (layer "F.Cu") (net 8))
 (segment (start 181.975735 52.775735) (end 181.924265 52.775735) (width 0.2) (layer "F.Cu") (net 8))
 (segment (start 184.7 55.5) (end 184.3 55.1) (width 0.2) (layer "F.Cu") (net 8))
 (segment (start 204.68125 50.125) (end 204.68125 52.81875) (width 0.2) (layer "F.Cu") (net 8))
 (segment (start 204.68125 52.81875) (end 203.9 53.6) (width 0.2) (layer "F.Cu") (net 8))
 (segment (start 184.3 55.1) (end 181.975735 52.775735) (width 0.2) (layer "F.Cu") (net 8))
 (via (at 186.7 55.5) (size 0.6) (drill 0.3) (layers "F.Cu" "B.Cu") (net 8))
 (via (at 181.924265 52.775735) (size 0.6) (drill 0.3) (layers "F.Cu" "B.Cu") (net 8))
 (via (at 203.9 53.6) (size 0.6) (drill 0.3) (layers "F.Cu" "B.Cu") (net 8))
 (segment (start 188.35825 53.84175) (end 186.7 55.5) (width 0.2) (layer "B.Cu") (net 8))
 (segment (start 203.9 53.6) (end 203.65825 53.84175) (width 0.2) (layer "B.Cu") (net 8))
 (segment (start 181.92125 52.77875) (end 178.61875 52.77875) (width 0.2) (layer "B.Cu") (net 8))
 (segment (start 181.924265 52.775735) (end 181.92125 52.77875) (width 0.2) (layer "B.Cu") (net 8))
 (segment (start 203.65825 53.84175) (end 188.35825 53.84175) (width 0.2) (layer "B.Cu") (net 8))
 (segment (start 185.21875 45.88125) (end 189.54425 41.55575) (width 0.2) (layer "F.Cu") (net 7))
 (segment (start 179.818748 49.9) (end 178.9575 49.9) (width 0.2) (layer "F.Cu") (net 7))
 (segment (start 185.21875 45.9) (end 185.21875 45.88125) (width 0.2) (layer "F.Cu") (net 7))
 (segment (start 189.54425 41.55575) (end 201.112 41.55575) (width 0.2) (layer "F.Cu") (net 7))
 (segment (start 201.112 41.55575) (end 204.68125 45.125) (width 0.2) (layer "F.Cu") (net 7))
 (segment (start 178.9575 49.9) (end 178.61875 50.23875) (width 0.2) (layer "F.Cu") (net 7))
 (via (at 179.818748 49.9) (size 0.6) (drill 0.3) (layers "F.Cu" "B.Cu") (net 7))
 (via (at 185.21875 45.9) (size 0.6) (drill 0.3) (layers "F.Cu" "B.Cu") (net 7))
 (segment (start 181.267479 48.432521) (end 181.267479 48.451269) (width 0.2) (layer "B.Cu") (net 7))
 (segment (start 185.21875 45.9) (end 183.8 45.9) (width 0.2) (layer "B.Cu") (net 7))
 (segment (start 181.267479 48.451269) (end 179.818748 49.9) (width 0.2) (layer "B.Cu") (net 7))
 (segment (start 183.8 45.9) (end 181.267479 48.432521) (width 0.2) (layer "B.Cu") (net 7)))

